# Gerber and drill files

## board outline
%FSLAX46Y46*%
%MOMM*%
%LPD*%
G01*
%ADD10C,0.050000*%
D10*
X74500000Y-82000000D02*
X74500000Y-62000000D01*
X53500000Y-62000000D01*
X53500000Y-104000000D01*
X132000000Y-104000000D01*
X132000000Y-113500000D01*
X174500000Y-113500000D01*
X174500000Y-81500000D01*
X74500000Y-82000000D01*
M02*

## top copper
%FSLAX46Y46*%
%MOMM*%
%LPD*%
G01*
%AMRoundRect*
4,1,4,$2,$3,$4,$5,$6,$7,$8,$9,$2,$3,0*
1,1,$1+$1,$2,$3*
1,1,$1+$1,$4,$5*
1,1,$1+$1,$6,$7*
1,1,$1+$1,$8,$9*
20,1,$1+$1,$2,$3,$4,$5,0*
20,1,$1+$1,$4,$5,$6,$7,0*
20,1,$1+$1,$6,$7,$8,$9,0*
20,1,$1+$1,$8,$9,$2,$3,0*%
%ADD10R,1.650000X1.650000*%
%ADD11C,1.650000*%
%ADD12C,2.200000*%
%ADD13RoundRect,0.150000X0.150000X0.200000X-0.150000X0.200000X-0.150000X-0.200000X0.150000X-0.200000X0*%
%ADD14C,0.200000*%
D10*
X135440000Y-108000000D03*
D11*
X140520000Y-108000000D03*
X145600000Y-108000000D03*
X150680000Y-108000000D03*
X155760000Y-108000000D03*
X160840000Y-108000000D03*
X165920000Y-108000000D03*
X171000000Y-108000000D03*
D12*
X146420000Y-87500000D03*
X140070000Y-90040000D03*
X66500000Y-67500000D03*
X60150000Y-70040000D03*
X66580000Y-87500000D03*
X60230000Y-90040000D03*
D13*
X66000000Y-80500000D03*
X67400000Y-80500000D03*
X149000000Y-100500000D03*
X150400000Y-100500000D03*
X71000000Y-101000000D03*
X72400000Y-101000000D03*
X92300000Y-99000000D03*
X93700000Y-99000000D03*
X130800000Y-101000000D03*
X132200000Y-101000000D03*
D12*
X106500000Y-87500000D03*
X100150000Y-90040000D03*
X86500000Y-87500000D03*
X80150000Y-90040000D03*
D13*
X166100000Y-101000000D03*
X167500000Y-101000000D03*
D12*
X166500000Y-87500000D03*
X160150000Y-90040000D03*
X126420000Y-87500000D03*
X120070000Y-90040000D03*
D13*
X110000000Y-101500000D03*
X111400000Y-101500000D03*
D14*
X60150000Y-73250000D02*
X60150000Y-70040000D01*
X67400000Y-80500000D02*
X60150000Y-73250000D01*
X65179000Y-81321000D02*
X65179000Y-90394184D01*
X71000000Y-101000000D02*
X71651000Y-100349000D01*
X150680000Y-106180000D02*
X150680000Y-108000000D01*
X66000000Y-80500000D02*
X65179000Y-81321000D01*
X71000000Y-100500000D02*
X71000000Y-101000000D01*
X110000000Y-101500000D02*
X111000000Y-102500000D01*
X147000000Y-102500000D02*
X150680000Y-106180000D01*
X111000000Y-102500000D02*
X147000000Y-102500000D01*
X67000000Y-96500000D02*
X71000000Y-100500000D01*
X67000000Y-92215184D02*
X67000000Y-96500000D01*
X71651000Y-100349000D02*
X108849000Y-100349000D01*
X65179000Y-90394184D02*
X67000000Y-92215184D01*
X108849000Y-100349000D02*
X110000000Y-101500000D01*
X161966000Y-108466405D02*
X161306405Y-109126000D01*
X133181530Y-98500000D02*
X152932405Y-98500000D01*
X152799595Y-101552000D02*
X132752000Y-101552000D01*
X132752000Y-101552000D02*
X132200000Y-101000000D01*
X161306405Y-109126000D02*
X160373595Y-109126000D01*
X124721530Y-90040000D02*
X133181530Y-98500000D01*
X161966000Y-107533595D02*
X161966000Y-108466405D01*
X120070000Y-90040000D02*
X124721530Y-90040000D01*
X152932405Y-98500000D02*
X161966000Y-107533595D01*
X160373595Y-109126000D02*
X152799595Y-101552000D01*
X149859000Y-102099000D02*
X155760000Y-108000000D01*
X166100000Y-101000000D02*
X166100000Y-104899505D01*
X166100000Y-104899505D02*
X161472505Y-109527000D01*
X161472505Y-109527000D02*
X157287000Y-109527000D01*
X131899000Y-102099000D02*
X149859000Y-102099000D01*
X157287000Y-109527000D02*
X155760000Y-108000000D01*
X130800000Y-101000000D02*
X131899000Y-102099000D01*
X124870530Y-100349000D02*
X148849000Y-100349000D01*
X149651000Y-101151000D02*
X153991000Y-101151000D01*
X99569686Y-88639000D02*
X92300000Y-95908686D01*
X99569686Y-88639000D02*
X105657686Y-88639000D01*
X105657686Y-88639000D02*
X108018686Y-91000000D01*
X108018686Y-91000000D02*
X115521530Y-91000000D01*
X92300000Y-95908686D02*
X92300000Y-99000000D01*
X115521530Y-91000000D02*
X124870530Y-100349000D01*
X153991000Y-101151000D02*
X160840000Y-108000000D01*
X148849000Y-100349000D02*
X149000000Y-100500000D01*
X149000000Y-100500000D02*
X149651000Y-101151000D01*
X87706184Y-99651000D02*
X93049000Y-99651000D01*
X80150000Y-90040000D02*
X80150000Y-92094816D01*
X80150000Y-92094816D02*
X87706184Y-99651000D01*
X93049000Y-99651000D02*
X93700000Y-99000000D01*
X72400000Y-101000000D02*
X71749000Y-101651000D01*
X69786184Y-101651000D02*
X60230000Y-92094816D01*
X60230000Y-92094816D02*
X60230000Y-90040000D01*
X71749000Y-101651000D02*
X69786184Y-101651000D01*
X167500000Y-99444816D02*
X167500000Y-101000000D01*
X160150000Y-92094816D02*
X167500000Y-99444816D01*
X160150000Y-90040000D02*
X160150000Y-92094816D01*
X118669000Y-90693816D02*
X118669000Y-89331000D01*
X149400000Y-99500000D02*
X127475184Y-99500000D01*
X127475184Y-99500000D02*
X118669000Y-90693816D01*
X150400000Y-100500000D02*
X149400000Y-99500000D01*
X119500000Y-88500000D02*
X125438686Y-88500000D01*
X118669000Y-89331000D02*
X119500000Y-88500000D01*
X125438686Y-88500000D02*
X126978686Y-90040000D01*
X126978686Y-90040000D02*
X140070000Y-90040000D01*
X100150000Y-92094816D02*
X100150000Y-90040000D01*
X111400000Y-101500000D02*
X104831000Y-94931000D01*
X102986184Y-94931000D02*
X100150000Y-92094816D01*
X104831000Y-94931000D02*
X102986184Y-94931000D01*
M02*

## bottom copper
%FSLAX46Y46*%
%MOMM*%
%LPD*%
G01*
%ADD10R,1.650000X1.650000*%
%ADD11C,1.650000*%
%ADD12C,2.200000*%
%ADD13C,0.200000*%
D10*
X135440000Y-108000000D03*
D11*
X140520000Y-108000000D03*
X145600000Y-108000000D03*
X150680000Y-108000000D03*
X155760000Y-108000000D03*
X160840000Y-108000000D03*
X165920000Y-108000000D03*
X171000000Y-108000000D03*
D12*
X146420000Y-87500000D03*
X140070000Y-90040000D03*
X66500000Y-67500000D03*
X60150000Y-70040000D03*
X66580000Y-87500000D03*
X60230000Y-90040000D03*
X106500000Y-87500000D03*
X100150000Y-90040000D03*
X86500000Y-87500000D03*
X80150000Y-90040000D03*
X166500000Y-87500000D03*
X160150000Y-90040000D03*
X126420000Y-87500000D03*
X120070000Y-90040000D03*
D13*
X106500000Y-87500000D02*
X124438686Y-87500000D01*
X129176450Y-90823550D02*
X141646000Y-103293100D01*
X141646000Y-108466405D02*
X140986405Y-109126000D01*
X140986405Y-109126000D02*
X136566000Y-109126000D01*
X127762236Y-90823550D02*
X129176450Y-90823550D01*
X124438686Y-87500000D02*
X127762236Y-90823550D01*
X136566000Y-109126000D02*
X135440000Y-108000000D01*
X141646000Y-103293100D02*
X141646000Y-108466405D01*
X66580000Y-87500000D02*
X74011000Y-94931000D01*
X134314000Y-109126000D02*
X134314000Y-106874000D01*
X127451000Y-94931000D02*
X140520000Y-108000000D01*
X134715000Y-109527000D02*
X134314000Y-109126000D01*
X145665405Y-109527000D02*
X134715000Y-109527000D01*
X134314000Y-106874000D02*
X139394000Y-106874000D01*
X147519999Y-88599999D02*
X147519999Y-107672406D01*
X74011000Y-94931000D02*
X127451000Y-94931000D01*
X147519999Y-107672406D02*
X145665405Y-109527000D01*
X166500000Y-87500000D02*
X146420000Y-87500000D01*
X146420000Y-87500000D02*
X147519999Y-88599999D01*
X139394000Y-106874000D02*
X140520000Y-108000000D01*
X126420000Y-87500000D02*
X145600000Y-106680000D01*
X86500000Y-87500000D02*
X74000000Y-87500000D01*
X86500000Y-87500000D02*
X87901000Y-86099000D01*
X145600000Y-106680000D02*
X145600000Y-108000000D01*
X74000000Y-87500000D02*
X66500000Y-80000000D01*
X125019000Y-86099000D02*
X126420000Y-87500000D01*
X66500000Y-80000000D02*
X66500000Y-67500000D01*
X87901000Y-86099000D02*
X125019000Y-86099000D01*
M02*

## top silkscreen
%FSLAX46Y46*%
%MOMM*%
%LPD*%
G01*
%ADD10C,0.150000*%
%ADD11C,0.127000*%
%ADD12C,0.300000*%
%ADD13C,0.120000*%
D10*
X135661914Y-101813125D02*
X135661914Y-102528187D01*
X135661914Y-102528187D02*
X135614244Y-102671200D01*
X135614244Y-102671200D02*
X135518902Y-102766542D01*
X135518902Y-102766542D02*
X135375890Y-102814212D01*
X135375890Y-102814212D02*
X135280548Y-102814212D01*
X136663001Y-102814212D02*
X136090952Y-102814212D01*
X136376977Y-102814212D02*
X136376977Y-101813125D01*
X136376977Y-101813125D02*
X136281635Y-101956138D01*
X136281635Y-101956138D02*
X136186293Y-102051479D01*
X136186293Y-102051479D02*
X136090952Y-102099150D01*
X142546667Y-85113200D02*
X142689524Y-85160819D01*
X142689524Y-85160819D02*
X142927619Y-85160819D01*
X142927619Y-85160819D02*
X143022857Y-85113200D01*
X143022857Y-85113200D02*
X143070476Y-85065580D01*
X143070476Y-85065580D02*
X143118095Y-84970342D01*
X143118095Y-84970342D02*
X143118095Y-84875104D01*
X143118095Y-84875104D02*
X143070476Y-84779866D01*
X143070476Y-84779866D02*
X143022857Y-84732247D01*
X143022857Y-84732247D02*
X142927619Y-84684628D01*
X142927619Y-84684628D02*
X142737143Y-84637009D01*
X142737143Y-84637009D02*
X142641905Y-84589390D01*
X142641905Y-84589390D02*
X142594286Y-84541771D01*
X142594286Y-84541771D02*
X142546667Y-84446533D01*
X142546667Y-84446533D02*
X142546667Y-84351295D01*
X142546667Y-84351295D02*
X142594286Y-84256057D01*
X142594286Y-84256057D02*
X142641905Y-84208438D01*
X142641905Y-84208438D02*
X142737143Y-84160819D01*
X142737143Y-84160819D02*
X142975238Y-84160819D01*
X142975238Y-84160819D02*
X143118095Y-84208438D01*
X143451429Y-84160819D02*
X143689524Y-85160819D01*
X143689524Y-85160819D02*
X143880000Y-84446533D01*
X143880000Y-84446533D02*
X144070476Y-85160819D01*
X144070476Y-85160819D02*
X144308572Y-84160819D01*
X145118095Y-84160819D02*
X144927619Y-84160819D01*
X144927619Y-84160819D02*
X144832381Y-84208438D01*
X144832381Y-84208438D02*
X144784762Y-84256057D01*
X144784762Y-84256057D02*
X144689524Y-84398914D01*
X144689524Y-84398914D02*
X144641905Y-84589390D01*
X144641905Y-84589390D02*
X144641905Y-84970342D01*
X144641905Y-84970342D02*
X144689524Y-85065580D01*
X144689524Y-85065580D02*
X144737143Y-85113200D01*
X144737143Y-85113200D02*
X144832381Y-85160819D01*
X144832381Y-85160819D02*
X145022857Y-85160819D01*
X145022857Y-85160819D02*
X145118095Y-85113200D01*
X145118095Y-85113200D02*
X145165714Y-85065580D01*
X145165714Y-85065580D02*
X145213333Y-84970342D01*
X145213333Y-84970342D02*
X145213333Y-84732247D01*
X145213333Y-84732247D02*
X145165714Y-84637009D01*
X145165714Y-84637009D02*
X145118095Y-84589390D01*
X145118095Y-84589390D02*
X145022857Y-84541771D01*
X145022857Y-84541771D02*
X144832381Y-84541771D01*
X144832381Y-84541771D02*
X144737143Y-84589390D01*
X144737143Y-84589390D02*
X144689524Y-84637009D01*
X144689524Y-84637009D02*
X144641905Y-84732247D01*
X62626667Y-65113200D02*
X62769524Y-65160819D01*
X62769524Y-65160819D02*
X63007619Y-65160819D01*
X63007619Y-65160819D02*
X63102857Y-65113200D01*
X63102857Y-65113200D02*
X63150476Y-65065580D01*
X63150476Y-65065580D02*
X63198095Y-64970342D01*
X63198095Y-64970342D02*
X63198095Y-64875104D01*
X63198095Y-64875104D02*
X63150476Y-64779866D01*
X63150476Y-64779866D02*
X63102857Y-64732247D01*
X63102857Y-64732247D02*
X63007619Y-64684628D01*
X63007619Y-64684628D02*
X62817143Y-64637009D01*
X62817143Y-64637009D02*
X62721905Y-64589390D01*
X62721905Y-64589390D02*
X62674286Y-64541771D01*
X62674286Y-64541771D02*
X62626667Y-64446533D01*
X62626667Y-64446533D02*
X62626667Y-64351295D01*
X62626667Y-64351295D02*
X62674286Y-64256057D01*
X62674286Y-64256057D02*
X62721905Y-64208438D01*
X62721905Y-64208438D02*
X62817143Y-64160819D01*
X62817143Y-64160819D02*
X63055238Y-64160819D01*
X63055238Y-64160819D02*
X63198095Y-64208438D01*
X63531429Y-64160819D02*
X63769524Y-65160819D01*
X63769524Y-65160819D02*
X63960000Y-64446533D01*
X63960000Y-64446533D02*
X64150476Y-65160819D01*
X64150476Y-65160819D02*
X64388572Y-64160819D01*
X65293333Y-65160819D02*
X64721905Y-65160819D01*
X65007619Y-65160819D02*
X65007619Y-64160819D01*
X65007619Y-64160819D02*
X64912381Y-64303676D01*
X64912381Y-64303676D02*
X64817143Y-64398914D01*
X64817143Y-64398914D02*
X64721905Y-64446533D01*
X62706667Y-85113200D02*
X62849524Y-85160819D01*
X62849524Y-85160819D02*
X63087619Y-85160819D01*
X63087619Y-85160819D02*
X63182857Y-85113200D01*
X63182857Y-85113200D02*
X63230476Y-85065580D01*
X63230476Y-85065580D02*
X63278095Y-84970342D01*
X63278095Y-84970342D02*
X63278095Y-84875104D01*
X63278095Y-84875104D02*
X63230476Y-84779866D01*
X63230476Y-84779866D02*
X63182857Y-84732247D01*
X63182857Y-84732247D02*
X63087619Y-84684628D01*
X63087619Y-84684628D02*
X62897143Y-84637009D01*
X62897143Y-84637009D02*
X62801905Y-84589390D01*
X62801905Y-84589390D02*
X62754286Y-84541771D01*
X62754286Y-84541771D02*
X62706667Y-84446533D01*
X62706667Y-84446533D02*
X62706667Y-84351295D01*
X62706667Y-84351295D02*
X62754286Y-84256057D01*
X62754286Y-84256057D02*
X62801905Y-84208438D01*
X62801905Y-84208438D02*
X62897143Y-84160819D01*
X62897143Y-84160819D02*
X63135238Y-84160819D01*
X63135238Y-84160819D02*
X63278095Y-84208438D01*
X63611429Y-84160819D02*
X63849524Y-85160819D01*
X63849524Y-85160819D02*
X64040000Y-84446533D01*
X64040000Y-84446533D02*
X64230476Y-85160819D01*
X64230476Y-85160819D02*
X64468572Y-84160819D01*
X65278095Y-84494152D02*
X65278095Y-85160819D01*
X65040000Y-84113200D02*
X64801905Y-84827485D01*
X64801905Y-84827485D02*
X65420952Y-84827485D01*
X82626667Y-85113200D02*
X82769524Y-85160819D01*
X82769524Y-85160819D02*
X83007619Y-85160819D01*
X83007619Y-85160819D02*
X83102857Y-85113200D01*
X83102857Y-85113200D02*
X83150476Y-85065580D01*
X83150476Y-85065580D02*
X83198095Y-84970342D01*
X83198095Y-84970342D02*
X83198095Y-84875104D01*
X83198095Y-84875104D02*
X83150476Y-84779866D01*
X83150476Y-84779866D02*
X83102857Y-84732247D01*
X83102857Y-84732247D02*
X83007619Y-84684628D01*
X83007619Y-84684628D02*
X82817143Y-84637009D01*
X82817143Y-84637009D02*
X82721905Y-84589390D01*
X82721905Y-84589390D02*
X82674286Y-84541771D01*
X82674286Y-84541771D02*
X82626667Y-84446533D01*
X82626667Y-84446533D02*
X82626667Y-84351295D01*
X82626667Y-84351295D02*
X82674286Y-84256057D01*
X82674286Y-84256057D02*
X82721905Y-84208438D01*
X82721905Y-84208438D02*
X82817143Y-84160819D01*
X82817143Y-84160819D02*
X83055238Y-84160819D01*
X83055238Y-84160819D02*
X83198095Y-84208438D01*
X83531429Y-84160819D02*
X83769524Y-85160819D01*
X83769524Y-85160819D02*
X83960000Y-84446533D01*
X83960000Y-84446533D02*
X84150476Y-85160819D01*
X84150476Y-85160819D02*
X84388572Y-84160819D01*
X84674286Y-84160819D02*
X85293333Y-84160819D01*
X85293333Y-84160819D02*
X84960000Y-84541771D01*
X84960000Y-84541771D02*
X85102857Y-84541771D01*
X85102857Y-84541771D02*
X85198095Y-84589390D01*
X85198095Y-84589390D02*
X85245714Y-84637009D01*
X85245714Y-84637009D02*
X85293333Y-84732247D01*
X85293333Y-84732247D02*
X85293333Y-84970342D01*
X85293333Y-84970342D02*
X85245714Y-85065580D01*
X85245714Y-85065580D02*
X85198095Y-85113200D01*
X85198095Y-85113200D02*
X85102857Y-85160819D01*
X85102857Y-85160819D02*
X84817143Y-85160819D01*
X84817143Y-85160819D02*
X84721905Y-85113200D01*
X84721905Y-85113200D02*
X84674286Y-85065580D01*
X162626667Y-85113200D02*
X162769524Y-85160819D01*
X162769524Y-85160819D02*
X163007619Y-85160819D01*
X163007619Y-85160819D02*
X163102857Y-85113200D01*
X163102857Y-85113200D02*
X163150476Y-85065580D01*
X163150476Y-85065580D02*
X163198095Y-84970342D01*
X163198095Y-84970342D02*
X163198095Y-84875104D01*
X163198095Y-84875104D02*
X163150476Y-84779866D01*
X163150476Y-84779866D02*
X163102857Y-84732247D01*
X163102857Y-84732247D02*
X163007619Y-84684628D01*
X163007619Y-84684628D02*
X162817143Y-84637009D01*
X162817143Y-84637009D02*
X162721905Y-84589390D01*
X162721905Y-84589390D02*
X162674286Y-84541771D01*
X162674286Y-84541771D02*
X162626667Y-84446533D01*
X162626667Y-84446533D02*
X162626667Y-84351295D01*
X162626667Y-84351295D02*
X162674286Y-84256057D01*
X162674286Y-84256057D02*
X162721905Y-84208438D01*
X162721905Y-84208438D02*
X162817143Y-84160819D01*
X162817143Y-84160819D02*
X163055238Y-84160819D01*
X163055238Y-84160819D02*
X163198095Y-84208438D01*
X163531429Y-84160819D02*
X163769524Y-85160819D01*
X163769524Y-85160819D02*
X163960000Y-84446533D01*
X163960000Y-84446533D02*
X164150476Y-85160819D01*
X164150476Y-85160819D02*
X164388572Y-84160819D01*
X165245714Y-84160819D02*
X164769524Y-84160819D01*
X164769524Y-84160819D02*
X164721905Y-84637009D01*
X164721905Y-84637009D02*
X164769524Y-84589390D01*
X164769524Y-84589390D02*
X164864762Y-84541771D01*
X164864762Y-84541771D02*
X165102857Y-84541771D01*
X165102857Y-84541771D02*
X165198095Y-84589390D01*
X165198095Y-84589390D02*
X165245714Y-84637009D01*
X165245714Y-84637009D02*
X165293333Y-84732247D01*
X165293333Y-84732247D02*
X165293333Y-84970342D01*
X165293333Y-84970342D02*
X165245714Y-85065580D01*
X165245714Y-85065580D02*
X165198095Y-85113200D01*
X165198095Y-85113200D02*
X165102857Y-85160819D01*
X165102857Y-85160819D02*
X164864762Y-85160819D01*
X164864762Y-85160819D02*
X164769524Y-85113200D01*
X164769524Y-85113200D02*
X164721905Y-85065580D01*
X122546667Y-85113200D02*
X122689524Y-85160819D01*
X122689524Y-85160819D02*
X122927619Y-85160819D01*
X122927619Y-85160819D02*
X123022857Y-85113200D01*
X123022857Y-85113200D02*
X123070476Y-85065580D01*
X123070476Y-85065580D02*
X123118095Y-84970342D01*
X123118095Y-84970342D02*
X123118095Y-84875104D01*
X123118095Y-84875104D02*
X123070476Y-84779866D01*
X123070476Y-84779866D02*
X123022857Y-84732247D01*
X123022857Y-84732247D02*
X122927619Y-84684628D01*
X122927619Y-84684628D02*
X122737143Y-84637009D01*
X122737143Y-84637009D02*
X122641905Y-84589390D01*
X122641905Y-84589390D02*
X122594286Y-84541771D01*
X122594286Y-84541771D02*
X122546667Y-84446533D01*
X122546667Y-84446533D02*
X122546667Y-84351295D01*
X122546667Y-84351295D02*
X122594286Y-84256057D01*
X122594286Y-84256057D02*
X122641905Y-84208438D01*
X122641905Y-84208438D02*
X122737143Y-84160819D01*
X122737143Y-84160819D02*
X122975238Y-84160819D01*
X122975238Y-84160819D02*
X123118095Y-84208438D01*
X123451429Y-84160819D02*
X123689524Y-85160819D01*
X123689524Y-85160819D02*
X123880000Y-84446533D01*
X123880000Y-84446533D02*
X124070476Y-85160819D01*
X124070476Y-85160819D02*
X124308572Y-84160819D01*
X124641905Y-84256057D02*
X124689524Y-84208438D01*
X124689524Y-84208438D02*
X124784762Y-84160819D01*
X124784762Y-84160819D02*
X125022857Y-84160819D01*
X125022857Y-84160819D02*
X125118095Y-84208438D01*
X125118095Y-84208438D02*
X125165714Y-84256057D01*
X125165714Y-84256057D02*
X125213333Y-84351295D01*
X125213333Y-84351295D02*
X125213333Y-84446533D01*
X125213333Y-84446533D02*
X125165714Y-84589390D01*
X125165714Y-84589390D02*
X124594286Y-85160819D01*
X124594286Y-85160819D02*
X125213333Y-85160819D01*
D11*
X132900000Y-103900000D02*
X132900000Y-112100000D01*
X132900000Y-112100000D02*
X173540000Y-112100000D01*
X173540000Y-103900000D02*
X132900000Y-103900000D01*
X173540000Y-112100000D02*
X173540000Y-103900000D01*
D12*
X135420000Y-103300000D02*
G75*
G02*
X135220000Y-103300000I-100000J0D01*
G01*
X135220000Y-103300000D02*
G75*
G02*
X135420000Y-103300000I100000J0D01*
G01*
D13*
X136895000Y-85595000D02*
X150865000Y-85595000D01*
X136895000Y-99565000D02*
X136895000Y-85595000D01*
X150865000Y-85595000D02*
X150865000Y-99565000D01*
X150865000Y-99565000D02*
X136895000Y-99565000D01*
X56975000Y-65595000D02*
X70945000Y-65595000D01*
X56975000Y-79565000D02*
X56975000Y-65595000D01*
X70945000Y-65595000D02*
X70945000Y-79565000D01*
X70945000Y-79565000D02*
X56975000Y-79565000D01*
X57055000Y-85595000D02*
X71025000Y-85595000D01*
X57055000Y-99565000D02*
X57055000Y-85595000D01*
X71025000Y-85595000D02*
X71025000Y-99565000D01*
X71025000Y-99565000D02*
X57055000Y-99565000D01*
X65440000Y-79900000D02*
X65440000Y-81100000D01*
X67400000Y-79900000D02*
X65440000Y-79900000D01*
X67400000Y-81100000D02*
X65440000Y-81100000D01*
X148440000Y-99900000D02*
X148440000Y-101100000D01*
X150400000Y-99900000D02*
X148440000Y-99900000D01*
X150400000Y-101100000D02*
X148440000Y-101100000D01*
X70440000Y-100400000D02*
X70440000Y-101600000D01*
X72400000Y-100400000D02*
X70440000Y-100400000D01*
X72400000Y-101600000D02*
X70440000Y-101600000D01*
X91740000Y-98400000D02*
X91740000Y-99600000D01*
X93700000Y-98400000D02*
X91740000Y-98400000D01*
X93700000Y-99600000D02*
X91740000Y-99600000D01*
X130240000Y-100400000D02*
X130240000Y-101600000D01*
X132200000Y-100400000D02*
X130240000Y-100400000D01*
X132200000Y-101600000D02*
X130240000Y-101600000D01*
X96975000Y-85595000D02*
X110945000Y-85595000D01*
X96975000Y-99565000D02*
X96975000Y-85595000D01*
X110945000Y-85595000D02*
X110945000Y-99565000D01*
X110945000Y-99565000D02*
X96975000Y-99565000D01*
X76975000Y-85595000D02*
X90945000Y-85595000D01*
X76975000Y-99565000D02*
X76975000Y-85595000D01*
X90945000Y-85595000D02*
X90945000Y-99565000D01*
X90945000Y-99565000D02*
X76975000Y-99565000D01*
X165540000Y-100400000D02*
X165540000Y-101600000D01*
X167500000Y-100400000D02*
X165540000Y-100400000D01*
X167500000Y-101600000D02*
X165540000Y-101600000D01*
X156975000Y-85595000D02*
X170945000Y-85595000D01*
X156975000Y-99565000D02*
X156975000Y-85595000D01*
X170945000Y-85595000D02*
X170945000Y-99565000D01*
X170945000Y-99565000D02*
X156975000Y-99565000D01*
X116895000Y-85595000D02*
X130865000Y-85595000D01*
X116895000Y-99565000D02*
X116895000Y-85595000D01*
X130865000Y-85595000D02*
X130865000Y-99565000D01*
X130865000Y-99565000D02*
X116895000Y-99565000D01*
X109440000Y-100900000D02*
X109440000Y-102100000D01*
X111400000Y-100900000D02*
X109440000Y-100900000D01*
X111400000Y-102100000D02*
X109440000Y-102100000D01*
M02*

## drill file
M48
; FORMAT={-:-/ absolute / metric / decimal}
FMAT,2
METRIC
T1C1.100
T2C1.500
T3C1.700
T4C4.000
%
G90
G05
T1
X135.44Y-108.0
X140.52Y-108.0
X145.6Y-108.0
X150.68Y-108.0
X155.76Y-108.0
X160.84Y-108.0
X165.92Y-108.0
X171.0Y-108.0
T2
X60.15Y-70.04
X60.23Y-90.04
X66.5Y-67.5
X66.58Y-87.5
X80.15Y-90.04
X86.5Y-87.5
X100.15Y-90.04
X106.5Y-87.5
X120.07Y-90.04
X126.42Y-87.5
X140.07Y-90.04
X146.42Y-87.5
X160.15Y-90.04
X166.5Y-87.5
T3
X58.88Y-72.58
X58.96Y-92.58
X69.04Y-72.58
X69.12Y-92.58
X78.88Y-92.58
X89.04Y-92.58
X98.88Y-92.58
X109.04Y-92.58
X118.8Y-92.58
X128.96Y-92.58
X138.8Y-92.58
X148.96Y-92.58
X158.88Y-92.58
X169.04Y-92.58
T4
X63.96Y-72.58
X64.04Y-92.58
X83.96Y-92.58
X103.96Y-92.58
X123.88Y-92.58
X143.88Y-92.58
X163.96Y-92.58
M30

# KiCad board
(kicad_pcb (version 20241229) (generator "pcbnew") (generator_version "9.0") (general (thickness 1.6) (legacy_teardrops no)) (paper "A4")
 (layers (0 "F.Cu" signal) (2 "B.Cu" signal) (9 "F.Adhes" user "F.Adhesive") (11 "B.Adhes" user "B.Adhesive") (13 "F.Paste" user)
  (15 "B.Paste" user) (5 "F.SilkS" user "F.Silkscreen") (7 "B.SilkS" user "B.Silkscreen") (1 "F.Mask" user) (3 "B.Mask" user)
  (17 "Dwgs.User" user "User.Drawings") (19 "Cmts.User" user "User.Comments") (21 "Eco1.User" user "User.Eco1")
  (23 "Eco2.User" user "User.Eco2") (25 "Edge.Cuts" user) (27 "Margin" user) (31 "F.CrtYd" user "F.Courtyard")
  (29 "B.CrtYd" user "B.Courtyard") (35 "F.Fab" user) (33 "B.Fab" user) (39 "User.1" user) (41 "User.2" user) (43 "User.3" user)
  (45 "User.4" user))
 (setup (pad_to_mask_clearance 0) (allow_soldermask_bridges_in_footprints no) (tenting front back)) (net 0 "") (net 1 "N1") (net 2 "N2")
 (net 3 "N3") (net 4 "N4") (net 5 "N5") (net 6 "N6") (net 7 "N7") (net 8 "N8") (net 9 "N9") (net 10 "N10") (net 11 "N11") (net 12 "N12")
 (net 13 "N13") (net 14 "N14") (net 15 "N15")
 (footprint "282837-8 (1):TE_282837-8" (layer "F.Cu") (at 135.44 108)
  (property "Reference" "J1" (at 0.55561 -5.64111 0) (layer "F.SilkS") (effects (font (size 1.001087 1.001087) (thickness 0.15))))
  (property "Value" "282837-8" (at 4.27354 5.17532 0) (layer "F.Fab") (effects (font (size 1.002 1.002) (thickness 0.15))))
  (fp_line (start -2.54 -4.1) (end -2.54 4.1) (stroke (width 0.127) (type solid)) (layer "F.SilkS"))
  (fp_line (start -2.54 4.1) (end 38.1 4.1) (stroke (width 0.127) (type solid)) (layer "F.SilkS"))
  (fp_line (start 38.1 -4.1) (end -2.54 -4.1) (stroke (width 0.127) (type solid)) (layer "F.SilkS"))
  (fp_line (start 38.1 4.1) (end 38.1 -4.1) (stroke (width 0.127) (type solid)) (layer "F.SilkS"))
  (fp_circle (center -0.12 -4.7) (end -0.02 -4.7) (stroke (width 0.3) (type solid)) (fill no) (layer "F.SilkS"))
  (pad "1" thru_hole rect (at 0 0) (size 1.65 1.65) (drill 1.1) (layers "*.Cu" "*.Mask") (remove_unused_layers no) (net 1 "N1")
   (solder_mask_margin 0.102))
  (pad "2" thru_hole circle (at 5.08 0) (size 1.65 1.65) (drill 1.1) (layers "*.Cu" "*.Mask") (remove_unused_layers no) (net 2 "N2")
   (solder_mask_margin 0.102))
  (pad "3" thru_hole circle (at 10.16 0) (size 1.65 1.65) (drill 1.1) (layers "*.Cu" "*.Mask") (remove_unused_layers no) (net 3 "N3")
   (solder_mask_margin 0.102))
  (pad "4" thru_hole circle (at 15.24 0) (size 1.65 1.65) (drill 1.1) (layers "*.Cu" "*.Mask") (remove_unused_layers no) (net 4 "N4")
   (solder_mask_margin 0.102))
  (pad "5" thru_hole circle (at 20.32 0) (size 1.65 1.65) (drill 1.1) (layers "*.Cu" "*.Mask") (remove_unused_layers no) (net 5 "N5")
   (solder_mask_margin 0.102))
  (pad "6" thru_hole circle (at 25.4 0) (size 1.65 1.65) (drill 1.1) (layers "*.Cu" "*.Mask") (remove_unused_layers no) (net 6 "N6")
   (solder_mask_margin 0.102))
  (pad "7" thru_hole circle (at 30.48 0) (size 1.65 1.65) (drill 1.1) (layers "*.Cu" "*.Mask") (remove_unused_layers no) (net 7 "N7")
   (solder_mask_margin 0.102))
  (pad "8" thru_hole circle (at 35.56 0) (size 1.65 1.65) (drill 1.1) (layers "*.Cu" "*.Mask") (remove_unused_layers no) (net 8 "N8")
   (solder_mask_margin 0.102)))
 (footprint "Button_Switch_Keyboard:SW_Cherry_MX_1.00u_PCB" (layer "F.Cu") (at 146.42 87.5)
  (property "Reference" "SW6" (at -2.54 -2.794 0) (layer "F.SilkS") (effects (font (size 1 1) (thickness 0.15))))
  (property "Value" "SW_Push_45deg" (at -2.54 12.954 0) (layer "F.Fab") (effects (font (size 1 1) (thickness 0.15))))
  (fp_line (start -9.525 -1.905) (end 4.445 -1.905) (stroke (width 0.12) (type solid)) (layer "F.SilkS"))
  (fp_line (start -9.525 12.065) (end -9.525 -1.905) (stroke (width 0.12) (type solid)) (layer "F.SilkS"))
  (fp_line (start 4.445 -1.905) (end 4.445 12.065) (stroke (width 0.12) (type solid)) (layer "F.SilkS"))
  (fp_line (start 4.445 12.065) (end -9.525 12.065) (stroke (width 0.12) (type solid)) (layer "F.SilkS"))
  (pad "" np_thru_hole circle (at -7.62 5.08) (size 1.7 1.7) (drill 1.7) (layers "*.Cu" "*.Mask"))
  (pad "" np_thru_hole circle (at -2.54 5.08) (size 4 4) (drill 4) (layers "*.Cu" "*.Mask"))
  (pad "" np_thru_hole circle (at 2.54 5.08) (size 1.7 1.7) (drill 1.7) (layers "*.Cu" "*.Mask"))
  (pad "1" thru_hole circle (at 0 0) (size 2.2 2.2) (drill 1.5) (layers "*.Cu" "*.Mask") (remove_unused_layers no) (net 2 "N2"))
  (pad "2" thru_hole circle (at -6.35 2.54) (size 2.2 2.2) (drill 1.5) (layers "*.Cu" "*.Mask") (remove_unused_layers no) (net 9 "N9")))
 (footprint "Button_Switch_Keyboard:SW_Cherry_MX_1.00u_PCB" (layer "F.Cu") (at 66.5 67.5)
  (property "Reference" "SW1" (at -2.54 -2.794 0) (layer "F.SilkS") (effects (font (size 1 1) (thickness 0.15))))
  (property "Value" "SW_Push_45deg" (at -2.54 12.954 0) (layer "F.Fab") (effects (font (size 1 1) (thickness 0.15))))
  (fp_line (start -9.525 -1.905) (end 4.445 -1.905) (stroke (width 0.12) (type solid)) (layer "F.SilkS"))
  (fp_line (start -9.525 12.065) (end -9.525 -1.905) (stroke (width 0.12) (type solid)) (layer "F.SilkS"))
  (fp_line (start 4.445 -1.905) (end 4.445 12.065) (stroke (width 0.12) (type solid)) (layer "F.SilkS"))
  (fp_line (start 4.445 12.065) (end -9.525 12.065) (stroke (width 0.12) (type solid)) (layer "F.SilkS"))
  (pad "" np_thru_hole circle (at -7.62 5.08) (size 1.7 1.7) (drill 1.7) (layers "*.Cu" "*.Mask"))
  (pad "" np_thru_hole circle (at -2.54 5.08) (size 4 4) (drill 4) (layers "*.Cu" "*.Mask"))
  (pad "" np_thru_hole circle (at 2.54 5.08) (size 1.7 1.7) (drill 1.7) (layers "*.Cu" "*.Mask"))
  (pad "1" thru_hole circle (at 0 0) (size 2.2 2.2) (drill 1.5) (layers "*.Cu" "*.Mask") (remove_unused_layers no) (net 3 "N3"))
  (pad "2" thru_hole circle (at -6.35 2.54) (size 2.2 2.2) (drill 1.5) (layers "*.Cu" "*.Mask") (remove_unused_layers no) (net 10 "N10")))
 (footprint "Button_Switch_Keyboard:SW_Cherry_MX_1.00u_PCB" (layer "F.Cu") (at 66.58 87.5)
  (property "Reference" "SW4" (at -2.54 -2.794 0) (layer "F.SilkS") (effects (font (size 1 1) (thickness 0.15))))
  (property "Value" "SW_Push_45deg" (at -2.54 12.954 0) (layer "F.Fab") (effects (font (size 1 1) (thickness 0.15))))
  (fp_line (start -9.525 -1.905) (end 4.445 -1.905) (stroke (width 0.12) (type solid)) (layer "F.SilkS"))
  (fp_line (start -9.525 12.065) (end -9.525 -1.905) (stroke (width 0.12) (type solid)) (layer "F.SilkS"))
  (fp_line (start 4.445 -1.905) (end 4.445 12.065) (stroke (width 0.12) (type solid)) (layer "F.SilkS"))
  (fp_line (start 4.445 12.065) (end -9.525 12.065) (stroke (width 0.12) (type solid)) (layer "F.SilkS"))
  (pad "" np_thru_hole circle (at -7.62 5.08) (size 1.7 1.7) (drill 1.7) (layers "*.Cu" "*.Mask"))
  (pad "" np_thru_hole circle (at -2.54 5.08) (size 4 4) (drill 4) (layers "*.Cu" "*.Mask"))
  (pad "" np_thru_hole circle (at 2.54 5.08) (size 1.7 1.7) (drill 1.7) (layers "*.Cu" "*.Mask"))
  (pad "1" thru_hole circle (at 0 0) (size 2.2 2.2) (drill 1.5) (layers "*.Cu" "*.Mask") (remove_unused_layers no) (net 2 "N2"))
  (pad "2" thru_hole circle (at -6.35 2.54) (size 2.2 2.2) (drill 1.5) (layers "*.Cu" "*.Mask") (remove_unused_layers no) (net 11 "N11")))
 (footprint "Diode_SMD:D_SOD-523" (layer "F.Cu") (at 66.7 80.5)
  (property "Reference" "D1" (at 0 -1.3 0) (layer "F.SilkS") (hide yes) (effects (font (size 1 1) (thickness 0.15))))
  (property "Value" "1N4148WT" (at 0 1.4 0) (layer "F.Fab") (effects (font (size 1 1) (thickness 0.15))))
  (fp_line (start -1.26 -0.6) (end -1.26 0.6) (stroke (width 0.12) (type solid)) (layer "F.SilkS"))
  (fp_line (start 0.7 -0.6) (end -1.26 -0.6) (stroke (width 0.12) (type solid)) (layer "F.SilkS"))
  (fp_line (start 0.7 0.6) (end -1.26 0.6) (stroke (width 0.12) (type solid)) (layer "F.SilkS"))
  (pad "1" smd roundrect (at -0.7 0 180) (size 0.6 0.7) (layers "F.Cu" "F.Mask" "F.Paste") (roundrect_rratio 0.25) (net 4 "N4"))
  (pad "2" smd roundrect (at 0.7 0 180) (size 0.6 0.7) (layers "F.Cu" "F.Mask" "F.Paste") (roundrect_rratio 0.25) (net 10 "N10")))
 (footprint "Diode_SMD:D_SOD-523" (layer "F.Cu") (at 149.7 100.5)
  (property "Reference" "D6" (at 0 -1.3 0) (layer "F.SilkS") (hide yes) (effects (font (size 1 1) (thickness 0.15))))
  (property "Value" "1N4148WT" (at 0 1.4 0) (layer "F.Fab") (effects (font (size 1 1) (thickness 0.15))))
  (fp_line (start -1.26 -0.6) (end -1.26 0.6) (stroke (width 0.12) (type solid)) (layer "F.SilkS"))
  (fp_line (start 0.7 -0.6) (end -1.26 -0.6) (stroke (width 0.12) (type solid)) (layer "F.SilkS"))
  (fp_line (start 0.7 0.6) (end -1.26 0.6) (stroke (width 0.12) (type solid)) (layer "F.SilkS"))
  (pad "1" smd roundrect (at -0.7 0 180) (size 0.6 0.7) (layers "F.Cu" "F.Mask" "F.Paste") (roundrect_rratio 0.25) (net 6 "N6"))
  (pad "2" smd roundrect (at 0.7 0 180) (size 0.6 0.7) (layers "F.Cu" "F.Mask" "F.Paste") (roundrect_rratio 0.25) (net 9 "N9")))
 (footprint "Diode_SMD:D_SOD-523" (layer "F.Cu") (at 71.7 101)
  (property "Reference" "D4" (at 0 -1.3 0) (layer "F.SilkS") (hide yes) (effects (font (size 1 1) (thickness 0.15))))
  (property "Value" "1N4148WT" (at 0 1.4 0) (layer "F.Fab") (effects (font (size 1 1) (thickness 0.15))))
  (fp_line (start -1.26 -0.6) (end -1.26 0.6) (stroke (width 0.12) (type solid)) (layer "F.SilkS"))
  (fp_line (start 0.7 -0.6) (end -1.26 -0.6) (stroke (width 0.12) (type solid)) (layer "F.SilkS"))
  (fp_line (start 0.7 0.6) (end -1.26 0.6) (stroke (width 0.12) (type solid)) (layer "F.SilkS"))
  (pad "1" smd roundrect (at -0.7 0 180) (size 0.6 0.7) (layers "F.Cu" "F.Mask" "F.Paste") (roundrect_rratio 0.25) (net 4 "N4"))
  (pad "2" smd roundrect (at 0.7 0 180) (size 0.6 0.7) (layers "F.Cu" "F.Mask" "F.Paste") (roundrect_rratio 0.25) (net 11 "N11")))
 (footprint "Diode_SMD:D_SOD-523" (layer "F.Cu") (at 93 99)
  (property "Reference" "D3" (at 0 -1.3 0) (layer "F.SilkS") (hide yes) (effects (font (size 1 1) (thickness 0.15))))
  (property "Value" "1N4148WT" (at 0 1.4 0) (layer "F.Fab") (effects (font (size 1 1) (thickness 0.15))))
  (fp_line (start -1.26 -0.6) (end -1.26 0.6) (stroke (width 0.12) (type solid)) (layer "F.SilkS"))
  (fp_line (start 0.7 -0.6) (end -1.26 -0.6) (stroke (width 0.12) (type solid)) (layer "F.SilkS"))
  (fp_line (start 0.7 0.6) (end -1.26 0.6) (stroke (width 0.12) (type solid)) (layer "F.SilkS"))
  (pad "1" smd roundrect (at -0.7 0 180) (size 0.6 0.7) (layers "F.Cu" "F.Mask" "F.Paste") (roundrect_rratio 0.25) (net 6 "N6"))
  (pad "2" smd roundrect (at 0.7 0 180) (size 0.6 0.7) (layers "F.Cu" "F.Mask" "F.Paste") (roundrect_rratio 0.25) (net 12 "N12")))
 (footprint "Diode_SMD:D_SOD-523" (layer "F.Cu") (at 131.5 101)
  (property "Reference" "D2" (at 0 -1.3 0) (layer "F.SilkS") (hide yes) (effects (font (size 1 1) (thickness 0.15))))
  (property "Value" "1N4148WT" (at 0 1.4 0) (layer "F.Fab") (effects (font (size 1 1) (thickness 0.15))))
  (fp_line (start -1.26 -0.6) (end -1.26 0.6) (stroke (width 0.12) (type solid)) (layer "F.SilkS"))
  (fp_line (start 0.7 -0.6) (end -1.26 -0.6) (stroke (width 0.12) (type solid)) (layer "F.SilkS"))
  (fp_line (start 0.7 0.6) (end -1.26 0.6) (stroke (width 0.12) (type solid)) (layer "F.SilkS"))
  (pad "1" smd roundrect (at -0.7 0 180) (size 0.6 0.7) (layers "F.Cu" "F.Mask" "F.Paste") (roundrect_rratio 0.25) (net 5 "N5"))
  (pad "2" smd roundrect (at 0.7 0 180) (size 0.6 0.7) (layers "F.Cu" "F.Mask" "F.Paste") (roundrect_rratio 0.25) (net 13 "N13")))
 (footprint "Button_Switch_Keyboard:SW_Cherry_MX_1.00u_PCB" (layer "F.Cu") (at 106.5 87.5)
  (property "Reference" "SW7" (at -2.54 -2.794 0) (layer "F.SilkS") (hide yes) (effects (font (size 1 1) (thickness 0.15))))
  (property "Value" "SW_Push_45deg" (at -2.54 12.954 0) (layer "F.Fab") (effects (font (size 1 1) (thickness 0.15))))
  (fp_line (start -9.525 -1.905) (end 4.445 -1.905) (stroke (width 0.12) (type solid)) (layer "F.SilkS"))
  (fp_line (start -9.525 12.065) (end -9.525 -1.905) (stroke (width 0.12) (type solid)) (layer "F.SilkS"))
  (fp_line (start 4.445 -1.905) (end 4.445 12.065) (stroke (width 0.12) (type solid)) (layer "F.SilkS"))
  (fp_line (start 4.445 12.065) (end -9.525 12.065) (stroke (width 0.12) (type solid)) (layer "F.SilkS"))
  (pad "" np_thru_hole circle (at -7.62 5.08) (size 1.7 1.7) (drill 1.7) (layers "*.Cu" "*.Mask"))
  (pad "" np_thru_hole circle (at -2.54 5.08) (size 4 4) (drill 4) (layers "*.Cu" "*.Mask"))
  (pad "" np_thru_hole circle (at 2.54 5.08) (size 1.7 1.7) (drill 1.7) (layers "*.Cu" "*.Mask"))
  (pad "1" thru_hole circle (at 0 0) (size 2.2 2.2) (drill 1.5) (layers "*.Cu" "*.Mask") (remove_unused_layers no) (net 1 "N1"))
  (pad "2" thru_hole circle (at -6.35 2.54) (size 2.2 2.2) (drill 1.5) (layers "*.Cu" "*.Mask") (remove_unused_layers no) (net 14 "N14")))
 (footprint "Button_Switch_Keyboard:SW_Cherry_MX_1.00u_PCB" (layer "F.Cu") (at 86.5 87.5)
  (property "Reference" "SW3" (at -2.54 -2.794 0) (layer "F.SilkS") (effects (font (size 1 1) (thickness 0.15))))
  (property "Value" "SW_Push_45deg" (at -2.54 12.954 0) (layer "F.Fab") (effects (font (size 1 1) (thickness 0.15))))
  (fp_line (start -9.525 -1.905) (end 4.445 -1.905) (stroke (width 0.12) (type solid)) (layer "F.SilkS"))
  (fp_line (start -9.525 12.065) (end -9.525 -1.905) (stroke (width 0.12) (type solid)) (layer "F.SilkS"))
  (fp_line (start 4.445 -1.905) (end 4.445 12.065) (stroke (width 0.12) (type solid)) (layer "F.SilkS"))
  (fp_line (start 4.445 12.065) (end -9.525 12.065) (stroke (width 0.12) (type solid)) (layer "F.SilkS"))
  (pad "" np_thru_hole circle (at -7.62 5.08) (size 1.7 1.7) (drill 1.7) (layers "*.Cu" "*.Mask"))
  (pad "" np_thru_hole circle (at -2.54 5.08) (size 4 4) (drill 4) (layers "*.Cu" "*.Mask"))
  (pad "" np_thru_hole circle (at 2.54 5.08) (size 1.7 1.7) (drill 1.7) (layers "*.Cu" "*.Mask"))
  (pad "1" thru_hole circle (at 0 0) (size 2.2 2.2) (drill 1.5) (layers "*.Cu" "*.Mask") (remove_unused_layers no) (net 3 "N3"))
  (pad "2" thru_hole circle (at -6.35 2.54) (size 2.2 2.2) (drill 1.5) (layers "*.Cu" "*.Mask") (remove_unused_layers no) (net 12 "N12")))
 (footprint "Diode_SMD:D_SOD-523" (layer "F.Cu") (at 166.8 101)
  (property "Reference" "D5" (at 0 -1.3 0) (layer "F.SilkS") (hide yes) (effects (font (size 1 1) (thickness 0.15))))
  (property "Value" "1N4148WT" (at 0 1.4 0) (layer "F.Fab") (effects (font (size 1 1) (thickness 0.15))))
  (fp_line (start -1.26 -0.6) (end -1.26 0.6) (stroke (width 0.12) (type solid)) (layer "F.SilkS"))
  (fp_line (start 0.7 -0.6) (end -1.26 -0.6) (stroke (width 0.12) (type solid)) (layer "F.SilkS"))
  (fp_line (start 0.7 0.6) (end -1.26 0.6) (stroke (width 0.12) (type solid)) (layer "F.SilkS"))
  (pad "1" smd roundrect (at -0.7 0 180) (size 0.6 0.7) (layers "F.Cu" "F.Mask" "F.Paste") (roundrect_rratio 0.25) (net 5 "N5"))
  (pad "2" smd roundrect (at 0.7 0 180) (size 0.6 0.7) (layers "F.Cu" "F.Mask" "F.Paste") (roundrect_rratio 0.25) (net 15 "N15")))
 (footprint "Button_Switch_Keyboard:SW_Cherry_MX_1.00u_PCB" (layer "F.Cu") (at 166.5 87.5)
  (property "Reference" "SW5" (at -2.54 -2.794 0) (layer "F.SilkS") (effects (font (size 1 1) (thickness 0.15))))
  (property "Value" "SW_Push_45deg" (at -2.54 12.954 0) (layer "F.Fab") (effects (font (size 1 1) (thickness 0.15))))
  (fp_line (start -9.525 -1.905) (end 4.445 -1.905) (stroke (width 0.12) (type solid)) (layer "F.SilkS"))
  (fp_line (start -9.525 12.065) (end -9.525 -1.905) (stroke (width 0.12) (type solid)) (layer "F.SilkS"))
  (fp_line (start 4.445 -1.905) (end 4.445 12.065) (stroke (width 0.12) (type solid)) (layer "F.SilkS"))
  (fp_line (start 4.445 12.065) (end -9.525 12.065) (stroke (width 0.12) (type solid)) (layer "F.SilkS"))
  (pad "" np_thru_hole circle (at -7.62 5.08) (size 1.7 1.7) (drill 1.7) (layers "*.Cu" "*.Mask"))
  (pad "" np_thru_hole circle (at -2.54 5.08) (size 4 4) (drill 4) (layers "*.Cu" "*.Mask"))
  (pad "" np_thru_hole circle (at 2.54 5.08) (size 1.7 1.7) (drill 1.7) (layers "*.Cu" "*.Mask"))
  (pad "1" thru_hole circle (at 0 0) (size 2.2 2.2) (drill 1.5) (layers "*.Cu" "*.Mask") (remove_unused_layers no) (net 2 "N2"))
  (pad "2" thru_hole circle (at -6.35 2.54) (size 2.2 2.2) (drill 1.5) (layers "*.Cu" "*.Mask") (remove_unused_layers no) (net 15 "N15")))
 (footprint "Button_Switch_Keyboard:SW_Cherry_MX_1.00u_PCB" (layer "F.Cu") (at 126.42 87.5)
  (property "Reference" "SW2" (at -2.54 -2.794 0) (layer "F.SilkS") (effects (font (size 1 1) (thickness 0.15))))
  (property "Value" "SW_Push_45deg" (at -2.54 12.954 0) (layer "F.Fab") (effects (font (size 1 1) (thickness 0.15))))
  (fp_line (start -9.525 -1.905) (end 4.445 -1.905) (stroke (width 0.12) (type solid)) (layer "F.SilkS"))
  (fp_line (start -9.525 12.065) (end -9.525 -1.905) (stroke (width 0.12) (type solid)) (layer "F.SilkS"))
  (fp_line (start 4.445 -1.905) (end 4.445 12.065) (stroke (width 0.12) (type solid)) (layer "F.SilkS"))
  (fp_line (start 4.445 12.065) (end -9.525 12.065) (stroke (width 0.12) (type solid)) (layer "F.SilkS"))
  (pad "" np_thru_hole circle (at -7.62 5.08) (size 1.7 1.7) (drill 1.7) (layers "*.Cu" "*.Mask"))
  (pad "" np_thru_hole circle (at -2.54 5.08) (size 4 4) (drill 4) (layers "*.Cu" "*.Mask"))
  (pad "" np_thru_hole circle (at 2.54 5.08) (size 1.7 1.7) (drill 1.7) (layers "*.Cu" "*.Mask"))
  (pad "1" thru_hole circle (at 0 0) (size 2.2 2.2) (drill 1.5) (layers "*.Cu" "*.Mask") (remove_unused_layers no) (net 3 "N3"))
  (pad "2" thru_hole circle (at -6.35 2.54) (size 2.2 2.2) (drill 1.5) (layers "*.Cu" "*.Mask") (remove_unused_layers no) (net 13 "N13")))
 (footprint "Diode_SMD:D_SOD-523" (layer "F.Cu") (at 110.7 101.5)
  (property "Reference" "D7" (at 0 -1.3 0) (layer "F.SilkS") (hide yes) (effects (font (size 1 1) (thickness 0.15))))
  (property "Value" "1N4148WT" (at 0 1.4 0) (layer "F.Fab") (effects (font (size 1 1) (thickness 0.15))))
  (fp_line (start -1.26 -0.6) (end -1.26 0.6) (stroke (width 0.12) (type solid)) (layer "F.SilkS"))
  (fp_line (start 0.7 -0.6) (end -1.26 -0.6) (stroke (width 0.12) (type solid)) (layer "F.SilkS"))
  (fp_line (start 0.7 0.6) (end -1.26 0.6) (stroke (width 0.12) (type solid)) (layer "F.SilkS"))
  (pad "1" smd roundrect (at -0.7 0 180) (size 0.6 0.7) (layers "F.Cu" "F.Mask" "F.Paste") (roundrect_rratio 0.25) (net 4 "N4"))
  (pad "2" smd roundrect (at 0.7 0 180) (size 0.6 0.7) (layers "F.Cu" "F.Mask" "F.Paste") (roundrect_rratio 0.25) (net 14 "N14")))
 (gr_poly
  (pts (xy 74.5 82) (xy 74.5 62) (xy 53.5 62) (xy 53.5 104) (xy 132 104) (xy 132 113.5) (xy 174.5 113.5) (xy 174.5 81.5))
  (stroke (width 0.05) (type solid)) (fill no) (layer "Edge.Cuts"))
 (segment (start 60.15 73.25) (end 60.15 70.04) (width 0.2) (layer "F.Cu") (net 10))
 (segment (start 67.4 80.5) (end 60.15 73.25) (width 0.2) (layer "F.Cu") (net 10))
 (segment (start 65.179 81.321) (end 65.179 90.394184) (width 0.2) (layer "F.Cu") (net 4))
 (segment (start 71 101) (end 71.651 100.349) (width 0.2) (layer "F.Cu") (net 4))
 (segment (start 150.68 106.18) (end 150.68 108) (width 0.2) (layer "F.Cu") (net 4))
 (segment (start 66 80.5) (end 65.179 81.321) (width 0.2) (layer "F.Cu") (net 4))
 (segment (start 71 100.5) (end 71 101) (width 0.2) (layer "F.Cu") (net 4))
 (segment (start 110 101.5) (end 111 102.5) (width 0.2) (layer "F.Cu") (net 4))
 (segment (start 147 102.5) (end 150.68 106.18) (width 0.2) (layer "F.Cu") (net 4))
 (segment (start 111 102.5) (end 147 102.5) (width 0.2) (layer "F.Cu") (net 4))
 (segment (start 67 96.5) (end 71 100.5) (width 0.2) (layer "F.Cu") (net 4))
 (segment (start 67 92.215184) (end 67 96.5) (width 0.2) (layer "F.Cu") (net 4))
 (segment (start 71.651 100.349) (end 108.849 100.349) (width 0.2) (layer "F.Cu") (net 4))
 (segment (start 65.179 90.394184) (end 67 92.215184) (width 0.2) (layer "F.Cu") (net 4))
 (segment (start 108.849 100.349) (end 110 101.5) (width 0.2) (layer "F.Cu") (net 4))
 (segment (start 161.966 108.466405) (end 161.306405 109.126) (width 0.2) (layer "F.Cu") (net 13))
 (segment (start 133.18153 98.5) (end 152.932405 98.5) (width 0.2) (layer "F.Cu") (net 13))
 (segment (start 152.799595 101.552) (end 132.752 101.552) (width 0.2) (layer "F.Cu") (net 13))
 (segment (start 132.752 101.552) (end 132.2 101) (width 0.2) (layer "F.Cu") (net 13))
 (segment (start 161.306405 109.126) (end 160.373595 109.126) (width 0.2) (layer "F.Cu") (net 13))
 (segment (start 124.72153 90.04) (end 133.18153 98.5) (width 0.2) (layer "F.Cu") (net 13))
 (segment (start 161.966 107.533595) (end 161.966 108.466405) (width 0.2) (layer "F.Cu") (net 13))
 (segment (start 120.07 90.04) (end 124.72153 90.04) (width 0.2) (layer "F.Cu") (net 13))
 (segment (start 152.932405 98.5) (end 161.966 107.533595) (width 0.2) (layer "F.Cu") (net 13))
 (segment (start 160.373595 109.126) (end 152.799595 101.552) (width 0.2) (layer "F.Cu") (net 13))
 (segment (start 149.859 102.099) (end 155.76 108) (width 0.2) (layer "F.Cu") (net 5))
 (segment (start 166.1 101) (end 166.1 104.899505) (width 0.2) (layer "F.Cu") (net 5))
 (segment (start 166.1 104.899505) (end 161.472505 109.527) (width 0.2) (layer "F.Cu") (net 5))
 (segment (start 161.472505 109.527) (end 157.287 109.527) (width 0.2) (layer "F.Cu") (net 5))
 (segment (start 131.899 102.099) (end 149.859 102.099) (width 0.2) (layer "F.Cu") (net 5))
 (segment (start 157.287 109.527) (end 155.76 108) (width 0.2) (layer "F.Cu") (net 5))
 (segment (start 130.8 101) (end 131.899 102.099) (width 0.2) (layer "F.Cu") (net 5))
 (segment (start 124.87053 100.349) (end 148.849 100.349) (width 0.2) (layer "F.Cu") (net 6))
 (segment (start 149.651 101.151) (end 153.991 101.151) (width 0.2) (layer "F.Cu") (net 6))
 (segment (start 99.569686 88.639) (end 92.3 95.908686) (width 0.2) (layer "F.Cu") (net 6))
 (segment (start 99.569686 88.639) (end 105.657686 88.639) (width 0.2) (layer "F.Cu") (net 6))
 (segment (start 105.657686 88.639) (end 108.018686 91) (width 0.2) (layer "F.Cu") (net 6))
 (segment (start 108.018686 91) (end 115.52153 91) (width 0.2) (layer "F.Cu") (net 6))
 (segment (start 92.3 95.908686) (end 92.3 99) (width 0.2) (layer "F.Cu") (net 6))
 (segment (start 115.52153 91) (end 124.87053 100.349) (width 0.2) (layer "F.Cu") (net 6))
 (segment (start 153.991 101.151) (end 160.84 108) (width 0.2) (layer "F.Cu") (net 6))
 (segment (start 148.849 100.349) (end 149 100.5) (width 0.2) (layer "F.Cu") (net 6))
 (segment (start 149 100.5) (end 149.651 101.151) (width 0.2) (layer "F.Cu") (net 6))
 (segment (start 87.706184 99.651) (end 93.049 99.651) (width 0.2) (layer "F.Cu") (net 12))
 (segment (start 80.15 90.04) (end 80.15 92.094816) (width 0.2) (layer "F.Cu") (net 12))
 (segment (start 80.15 92.094816) (end 87.706184 99.651) (width 0.2) (layer "F.Cu") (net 12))
 (segment (start 93.049 99.651) (end 93.7 99) (width 0.2) (layer "F.Cu") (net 12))
 (segment (start 72.4 101) (end 71.749 101.651) (width 0.2) (layer "F.Cu") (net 11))
 (segment (start 69.786184 101.651) (end 60.23 92.094816) (width 0.2) (layer "F.Cu") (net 11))
 (segment (start 60.23 92.094816) (end 60.23 90.04) (width 0.2) (layer "F.Cu") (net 11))
 (segment (start 71.749 101.651) (end 69.786184 101.651) (width 0.2) (layer "F.Cu") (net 11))
 (segment (start 167.5 99.444816) (end 167.5 101) (width 0.2) (layer "F.Cu") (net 15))
 (segment (start 160.15 92.094816) (end 167.5 99.444816) (width 0.2) (layer "F.Cu") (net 15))
 (segment (start 160.15 90.04) (end 160.15 92.094816) (width 0.2) (layer "F.Cu") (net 15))
 (segment (start 118.669 90.693816) (end 118.669 89.331) (width 0.2) (layer "F.Cu") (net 9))
 (segment (start 149.4 99.5) (end 127.475184 99.5) (width 0.2) (layer "F.Cu") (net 9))
 (segment (start 127.475184 99.5) (end 118.669 90.693816) (width 0.2) (layer "F.Cu") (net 9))
 (segment (start 150.4 100.5) (end 149.4 99.5) (width 0.2) (layer "F.Cu") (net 9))
 (segment (start 119.5 88.5) (end 125.438686 88.5) (width 0.2) (layer "F.Cu") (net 9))
 (segment (start 118.669 89.331) (end 119.5 88.5) (width 0.2) (layer "F.Cu") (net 9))
 (segment (start 125.438686 88.5) (end 126.978686 90.04) (width 0.2) (layer "F.Cu") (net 9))
 (segment (start 126.978686 90.04) (end 140.07 90.04) (width 0.2) (layer "F.Cu") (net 9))
 (segment (start 100.15 92.094816) (end 100.15 90.04) (width 0.2) (layer "F.Cu") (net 14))
 (segment (start 111.4 101.5) (end 104.831 94.931) (width 0.2) (layer "F.Cu") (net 14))
 (segment (start 102.986184 94.931) (end 100.15 92.094816) (width 0.2) (layer "F.Cu") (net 14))
 (segment (start 104.831 94.931) (end 102.986184 94.931) (width 0.2) (layer "F.Cu") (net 14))
 (segment (start 106.5 87.5) (end 124.438686 87.5) (width 0.2) (layer "B.Cu") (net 1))
 (segment (start 129.17645 90.82355) (end 141.646 103.2931) (width 0.2) (layer "B.Cu") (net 1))
 (segment (start 141.646 108.466405) (end 140.986405 109.126) (width 0.2) (layer "B.Cu") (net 1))
 (segment (start 140.986405 109.126) (end 136.566 109.126) (width 0.2) (layer "B.Cu") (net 1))
 (segment (start 127.762236 90.82355) (end 129.17645 90.82355) (width 0.2) (layer "B.Cu") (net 1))
 (segment (start 124.438686 87.5) (end 127.762236 90.82355) (width 0.2) (layer "B.Cu") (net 1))
 (segment (start 136.566 109.126) (end 135.44 108) (width 0.2) (layer "B.Cu") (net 1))
 (segment (start 141.646 103.2931) (end 141.646 108.466405) (width 0.2) (layer "B.Cu") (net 1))
 (segment (start 66.58 87.5) (end 74.011 94.931) (width 0.2) (layer "B.Cu") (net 2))
 (segment (start 134.314 109.126) (end 134.314 106.874) (width 0.2) (layer "B.Cu") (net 2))
 (segment (start 127.451 94.931) (end 140.52 108) (width 0.2) (layer "B.Cu") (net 2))
 (segment (start 134.715 109.527) (end 134.314 109.126) (width 0.2) (layer "B.Cu") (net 2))
 (segment (start 145.665405 109.527) (end 134.715 109.527) (width 0.2) (layer "B.Cu") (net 2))
 (segment (start 134.314 106.874) (end 139.394 106.874) (width 0.2) (layer "B.Cu") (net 2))
 (segment (start 147.519999 88.599999) (end 147.519999 107.672406) (width 0.2) (layer "B.Cu") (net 2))
 (segment (start 74.011 94.931) (end 127.451 94.931) (width 0.2) (layer "B.Cu") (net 2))
 (segment (start 147.519999 107.672406) (end 145.665405 109.527) (width 0.2) (layer "B.Cu") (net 2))
 (segment (start 166.5 87.5) (end 146.42 87.5) (width 0.2) (layer "B.Cu") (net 2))
 (segment (start 146.42 87.5) (end 147.519999 88.599999) (width 0.2) (layer "B.Cu") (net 2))
 (segment (start 139.394 106.874) (end 140.52 108) (width 0.2) (layer "B.Cu") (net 2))
 (segment (start 126.42 87.5) (end 145.6 106.68) (width 0.2) (layer "B.Cu") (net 3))
 (segment (start 86.5 87.5) (end 74 87.5) (width 0.2) (layer "B.Cu") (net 3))
 (segment (start 86.5 87.5) (end 87.901 86.099) (width 0.2) (layer "B.Cu") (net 3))
 (segment (start 145.6 106.68) (end 145.6 108) (width 0.2) (layer "B.Cu") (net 3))
 (segment (start 74 87.5) (end 66.5 80) (width 0.2) (layer "B.Cu") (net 3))
 (segment (start 125.019 86.099) (end 126.42 87.5) (width 0.2) (layer "B.Cu") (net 3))
 (segment (start 66.5 80) (end 66.5 67.5) (width 0.2) (layer "B.Cu") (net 3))
 (segment (start 87.901 86.099) (end 125.019 86.099) (width 0.2) (layer "B.Cu") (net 3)))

